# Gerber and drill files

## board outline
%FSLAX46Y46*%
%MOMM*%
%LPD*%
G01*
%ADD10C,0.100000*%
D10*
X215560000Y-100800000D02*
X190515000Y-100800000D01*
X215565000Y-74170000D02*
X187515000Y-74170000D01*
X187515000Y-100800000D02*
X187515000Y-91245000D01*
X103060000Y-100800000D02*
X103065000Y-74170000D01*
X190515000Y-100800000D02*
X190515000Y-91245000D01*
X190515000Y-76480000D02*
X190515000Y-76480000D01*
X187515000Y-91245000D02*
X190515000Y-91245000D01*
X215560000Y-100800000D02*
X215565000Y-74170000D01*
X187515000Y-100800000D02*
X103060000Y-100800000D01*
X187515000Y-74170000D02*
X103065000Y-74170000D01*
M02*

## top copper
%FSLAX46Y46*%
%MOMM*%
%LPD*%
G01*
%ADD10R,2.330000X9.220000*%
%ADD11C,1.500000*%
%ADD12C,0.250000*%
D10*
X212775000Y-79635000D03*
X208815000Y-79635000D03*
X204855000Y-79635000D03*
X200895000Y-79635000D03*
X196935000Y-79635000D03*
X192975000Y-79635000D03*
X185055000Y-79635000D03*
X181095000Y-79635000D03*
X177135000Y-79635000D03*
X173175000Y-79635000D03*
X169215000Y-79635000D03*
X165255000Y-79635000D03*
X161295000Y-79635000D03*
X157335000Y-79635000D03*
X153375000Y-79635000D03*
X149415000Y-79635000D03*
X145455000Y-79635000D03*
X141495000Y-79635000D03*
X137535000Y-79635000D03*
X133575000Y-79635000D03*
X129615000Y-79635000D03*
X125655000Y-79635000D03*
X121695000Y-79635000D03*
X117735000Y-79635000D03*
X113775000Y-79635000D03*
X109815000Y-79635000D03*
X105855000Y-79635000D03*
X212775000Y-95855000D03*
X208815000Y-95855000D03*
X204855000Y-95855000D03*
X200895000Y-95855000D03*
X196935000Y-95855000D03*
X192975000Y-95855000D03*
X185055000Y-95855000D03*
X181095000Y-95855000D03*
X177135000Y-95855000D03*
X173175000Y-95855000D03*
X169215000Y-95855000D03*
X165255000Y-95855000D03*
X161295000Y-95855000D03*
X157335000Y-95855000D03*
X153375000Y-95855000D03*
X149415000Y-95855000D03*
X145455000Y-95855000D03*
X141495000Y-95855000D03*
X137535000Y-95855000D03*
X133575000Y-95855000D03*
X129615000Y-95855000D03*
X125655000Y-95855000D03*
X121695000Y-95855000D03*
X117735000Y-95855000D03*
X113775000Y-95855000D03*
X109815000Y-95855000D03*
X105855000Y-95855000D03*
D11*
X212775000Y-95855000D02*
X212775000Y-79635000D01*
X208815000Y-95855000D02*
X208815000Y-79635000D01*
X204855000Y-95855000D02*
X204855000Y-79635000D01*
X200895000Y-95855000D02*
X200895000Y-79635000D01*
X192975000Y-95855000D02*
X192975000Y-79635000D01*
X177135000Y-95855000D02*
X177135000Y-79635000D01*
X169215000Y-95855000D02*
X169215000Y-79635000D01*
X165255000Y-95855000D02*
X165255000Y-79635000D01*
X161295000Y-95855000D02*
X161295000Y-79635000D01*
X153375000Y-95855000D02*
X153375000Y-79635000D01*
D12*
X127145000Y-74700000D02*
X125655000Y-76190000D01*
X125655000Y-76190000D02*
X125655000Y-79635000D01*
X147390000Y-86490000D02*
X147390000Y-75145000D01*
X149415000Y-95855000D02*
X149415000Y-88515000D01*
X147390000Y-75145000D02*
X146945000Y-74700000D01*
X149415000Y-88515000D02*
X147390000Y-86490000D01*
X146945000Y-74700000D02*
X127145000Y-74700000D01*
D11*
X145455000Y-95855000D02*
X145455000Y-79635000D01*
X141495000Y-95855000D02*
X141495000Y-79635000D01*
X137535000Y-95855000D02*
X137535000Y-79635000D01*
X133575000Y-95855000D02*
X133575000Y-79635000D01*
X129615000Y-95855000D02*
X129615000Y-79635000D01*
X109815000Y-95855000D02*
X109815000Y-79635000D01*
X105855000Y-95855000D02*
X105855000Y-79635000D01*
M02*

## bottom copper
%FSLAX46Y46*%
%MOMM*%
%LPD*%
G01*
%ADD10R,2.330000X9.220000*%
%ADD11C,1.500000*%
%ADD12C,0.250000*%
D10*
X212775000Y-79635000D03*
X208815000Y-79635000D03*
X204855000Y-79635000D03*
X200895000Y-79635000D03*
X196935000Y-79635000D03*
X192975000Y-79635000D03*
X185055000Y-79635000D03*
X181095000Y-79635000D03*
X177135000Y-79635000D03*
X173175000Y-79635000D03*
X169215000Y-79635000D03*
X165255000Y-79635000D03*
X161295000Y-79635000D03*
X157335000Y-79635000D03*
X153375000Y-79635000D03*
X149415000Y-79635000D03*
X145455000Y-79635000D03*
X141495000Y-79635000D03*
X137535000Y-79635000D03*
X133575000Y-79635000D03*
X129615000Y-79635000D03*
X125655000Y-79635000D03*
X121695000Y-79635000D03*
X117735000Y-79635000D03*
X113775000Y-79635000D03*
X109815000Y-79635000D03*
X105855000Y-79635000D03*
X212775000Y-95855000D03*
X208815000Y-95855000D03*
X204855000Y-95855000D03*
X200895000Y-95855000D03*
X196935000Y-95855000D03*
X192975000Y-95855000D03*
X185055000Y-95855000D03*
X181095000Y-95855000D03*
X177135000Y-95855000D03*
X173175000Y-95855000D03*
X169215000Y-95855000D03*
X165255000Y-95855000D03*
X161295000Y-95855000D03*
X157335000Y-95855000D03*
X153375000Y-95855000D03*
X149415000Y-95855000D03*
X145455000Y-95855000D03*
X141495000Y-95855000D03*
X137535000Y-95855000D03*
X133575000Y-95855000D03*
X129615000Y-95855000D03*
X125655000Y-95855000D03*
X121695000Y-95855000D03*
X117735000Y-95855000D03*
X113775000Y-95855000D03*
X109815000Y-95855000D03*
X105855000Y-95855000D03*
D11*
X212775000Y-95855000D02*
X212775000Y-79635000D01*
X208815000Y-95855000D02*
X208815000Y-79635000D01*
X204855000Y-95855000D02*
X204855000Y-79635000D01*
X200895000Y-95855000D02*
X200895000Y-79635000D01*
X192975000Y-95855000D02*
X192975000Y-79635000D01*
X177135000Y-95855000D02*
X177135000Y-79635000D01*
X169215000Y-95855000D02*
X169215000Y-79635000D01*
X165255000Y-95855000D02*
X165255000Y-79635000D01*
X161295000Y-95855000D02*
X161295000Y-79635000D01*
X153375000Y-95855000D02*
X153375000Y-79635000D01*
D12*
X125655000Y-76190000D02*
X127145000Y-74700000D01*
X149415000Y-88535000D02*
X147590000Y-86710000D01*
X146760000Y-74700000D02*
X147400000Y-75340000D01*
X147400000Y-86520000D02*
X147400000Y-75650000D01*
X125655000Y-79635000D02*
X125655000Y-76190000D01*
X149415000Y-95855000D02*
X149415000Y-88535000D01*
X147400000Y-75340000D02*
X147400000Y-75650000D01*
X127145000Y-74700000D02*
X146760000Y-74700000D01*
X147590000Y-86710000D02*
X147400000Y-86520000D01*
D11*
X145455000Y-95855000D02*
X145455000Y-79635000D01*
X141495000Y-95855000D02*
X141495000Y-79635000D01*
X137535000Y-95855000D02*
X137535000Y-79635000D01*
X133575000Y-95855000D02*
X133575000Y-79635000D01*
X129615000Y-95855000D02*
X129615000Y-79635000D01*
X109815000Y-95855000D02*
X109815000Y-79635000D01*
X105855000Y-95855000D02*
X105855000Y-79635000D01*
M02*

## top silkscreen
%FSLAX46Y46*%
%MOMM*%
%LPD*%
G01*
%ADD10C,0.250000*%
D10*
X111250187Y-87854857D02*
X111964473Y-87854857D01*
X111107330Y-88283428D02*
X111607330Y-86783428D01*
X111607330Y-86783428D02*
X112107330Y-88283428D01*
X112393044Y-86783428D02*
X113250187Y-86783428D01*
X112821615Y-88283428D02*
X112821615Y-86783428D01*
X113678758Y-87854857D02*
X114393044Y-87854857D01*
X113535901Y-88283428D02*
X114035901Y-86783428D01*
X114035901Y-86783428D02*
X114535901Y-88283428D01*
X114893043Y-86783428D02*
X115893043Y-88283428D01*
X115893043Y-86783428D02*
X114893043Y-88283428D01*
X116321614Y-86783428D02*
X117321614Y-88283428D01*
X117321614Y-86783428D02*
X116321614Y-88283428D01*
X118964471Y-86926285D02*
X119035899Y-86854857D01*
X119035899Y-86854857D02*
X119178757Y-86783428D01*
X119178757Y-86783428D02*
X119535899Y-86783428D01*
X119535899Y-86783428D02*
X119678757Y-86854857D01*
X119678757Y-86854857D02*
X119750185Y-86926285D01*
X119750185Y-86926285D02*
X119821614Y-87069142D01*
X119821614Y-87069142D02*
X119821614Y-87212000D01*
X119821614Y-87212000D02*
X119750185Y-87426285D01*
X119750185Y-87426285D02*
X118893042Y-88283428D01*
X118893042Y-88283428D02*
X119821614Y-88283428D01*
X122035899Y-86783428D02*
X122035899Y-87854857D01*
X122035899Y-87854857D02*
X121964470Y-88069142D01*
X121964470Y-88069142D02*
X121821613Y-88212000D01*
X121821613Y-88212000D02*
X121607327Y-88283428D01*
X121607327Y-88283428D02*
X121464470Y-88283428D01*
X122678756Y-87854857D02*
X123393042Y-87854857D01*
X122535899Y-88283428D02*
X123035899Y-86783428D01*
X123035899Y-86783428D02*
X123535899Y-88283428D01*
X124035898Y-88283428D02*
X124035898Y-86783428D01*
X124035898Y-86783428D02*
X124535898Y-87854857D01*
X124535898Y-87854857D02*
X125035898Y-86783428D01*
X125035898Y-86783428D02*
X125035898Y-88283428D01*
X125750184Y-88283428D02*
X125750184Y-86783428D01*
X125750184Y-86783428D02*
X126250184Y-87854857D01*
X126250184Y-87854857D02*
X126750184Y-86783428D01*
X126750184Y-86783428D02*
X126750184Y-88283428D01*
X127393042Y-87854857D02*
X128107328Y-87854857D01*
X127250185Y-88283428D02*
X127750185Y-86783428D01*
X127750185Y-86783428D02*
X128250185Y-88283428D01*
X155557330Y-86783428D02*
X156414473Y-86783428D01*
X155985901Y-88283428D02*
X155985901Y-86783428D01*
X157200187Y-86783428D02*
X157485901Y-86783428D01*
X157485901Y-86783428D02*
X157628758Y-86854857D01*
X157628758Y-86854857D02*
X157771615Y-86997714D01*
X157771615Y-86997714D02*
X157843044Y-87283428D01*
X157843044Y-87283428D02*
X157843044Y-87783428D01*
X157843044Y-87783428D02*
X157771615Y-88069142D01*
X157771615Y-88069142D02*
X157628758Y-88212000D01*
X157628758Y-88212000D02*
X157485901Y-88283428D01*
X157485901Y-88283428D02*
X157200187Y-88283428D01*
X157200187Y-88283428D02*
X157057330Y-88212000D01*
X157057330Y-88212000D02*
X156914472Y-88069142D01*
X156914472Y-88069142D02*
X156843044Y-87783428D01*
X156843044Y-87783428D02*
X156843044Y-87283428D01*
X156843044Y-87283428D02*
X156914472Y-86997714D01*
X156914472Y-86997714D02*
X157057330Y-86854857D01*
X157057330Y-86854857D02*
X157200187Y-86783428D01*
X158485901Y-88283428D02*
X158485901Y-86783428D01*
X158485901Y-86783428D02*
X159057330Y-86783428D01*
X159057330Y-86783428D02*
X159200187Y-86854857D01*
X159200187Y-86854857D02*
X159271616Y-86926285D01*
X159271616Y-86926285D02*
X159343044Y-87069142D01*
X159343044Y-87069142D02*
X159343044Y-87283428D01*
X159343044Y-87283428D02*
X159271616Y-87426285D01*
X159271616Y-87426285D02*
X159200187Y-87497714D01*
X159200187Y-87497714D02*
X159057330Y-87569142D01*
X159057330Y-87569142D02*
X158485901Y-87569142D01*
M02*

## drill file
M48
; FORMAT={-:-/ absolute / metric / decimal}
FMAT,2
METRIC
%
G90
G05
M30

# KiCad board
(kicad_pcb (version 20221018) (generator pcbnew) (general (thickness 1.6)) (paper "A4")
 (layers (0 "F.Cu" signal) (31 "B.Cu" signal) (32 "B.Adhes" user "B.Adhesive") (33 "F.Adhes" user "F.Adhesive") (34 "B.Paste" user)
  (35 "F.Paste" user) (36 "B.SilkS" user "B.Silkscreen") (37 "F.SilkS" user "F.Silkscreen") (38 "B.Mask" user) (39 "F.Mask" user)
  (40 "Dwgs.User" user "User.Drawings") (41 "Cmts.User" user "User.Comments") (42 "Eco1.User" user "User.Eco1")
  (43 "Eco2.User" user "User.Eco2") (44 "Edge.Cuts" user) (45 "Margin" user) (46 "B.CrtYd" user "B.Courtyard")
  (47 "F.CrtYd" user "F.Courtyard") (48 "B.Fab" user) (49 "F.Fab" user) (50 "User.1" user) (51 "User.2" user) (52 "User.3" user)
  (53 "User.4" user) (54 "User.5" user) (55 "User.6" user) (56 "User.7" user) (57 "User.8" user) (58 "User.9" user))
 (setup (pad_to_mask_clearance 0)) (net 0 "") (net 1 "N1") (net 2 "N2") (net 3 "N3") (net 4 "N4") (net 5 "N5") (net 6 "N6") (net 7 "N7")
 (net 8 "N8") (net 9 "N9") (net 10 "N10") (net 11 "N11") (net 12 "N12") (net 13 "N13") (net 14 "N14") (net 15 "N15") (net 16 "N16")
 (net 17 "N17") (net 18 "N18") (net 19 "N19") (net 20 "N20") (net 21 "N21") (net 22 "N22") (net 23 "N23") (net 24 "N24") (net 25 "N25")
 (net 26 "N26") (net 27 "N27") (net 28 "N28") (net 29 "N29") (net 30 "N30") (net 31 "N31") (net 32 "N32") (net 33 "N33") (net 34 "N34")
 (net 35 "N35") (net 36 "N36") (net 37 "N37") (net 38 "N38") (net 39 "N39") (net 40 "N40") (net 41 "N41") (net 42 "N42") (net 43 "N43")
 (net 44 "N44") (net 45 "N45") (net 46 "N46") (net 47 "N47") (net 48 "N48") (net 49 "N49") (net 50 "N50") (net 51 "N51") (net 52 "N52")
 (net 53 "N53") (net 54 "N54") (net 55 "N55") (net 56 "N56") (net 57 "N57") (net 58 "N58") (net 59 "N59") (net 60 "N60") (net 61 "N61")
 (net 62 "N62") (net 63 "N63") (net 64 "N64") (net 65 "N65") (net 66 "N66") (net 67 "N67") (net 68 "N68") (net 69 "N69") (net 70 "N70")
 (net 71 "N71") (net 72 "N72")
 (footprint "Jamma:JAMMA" (layer "F.Cu") (at 159.435 79.635 180)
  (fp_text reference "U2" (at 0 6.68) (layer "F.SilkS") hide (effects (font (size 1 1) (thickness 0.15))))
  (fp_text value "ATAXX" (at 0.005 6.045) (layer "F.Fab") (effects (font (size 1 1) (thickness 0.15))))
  (pad "1" smd rect (at -53.34 0 180) (size 2.33 9.22) (layers "F.Cu" "F.Paste" "F.Mask") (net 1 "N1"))
  (pad "2" smd rect (at -49.38 0 180) (size 2.33 9.22) (layers "F.Cu" "F.Paste" "F.Mask") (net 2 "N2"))
  (pad "3" smd rect (at -45.42 0 180) (size 2.33 9.22) (layers "F.Cu" "F.Paste" "F.Mask") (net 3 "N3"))
  (pad "4" smd rect (at -41.46 0 180) (size 2.33 9.22) (layers "F.Cu" "F.Paste" "F.Mask") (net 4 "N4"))
  (pad "5" smd rect (at -37.5 0 180) (size 2.33 9.22) (layers "F.Cu" "F.Paste" "F.Mask") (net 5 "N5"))
  (pad "6" smd rect (at -33.54 0 180) (size 2.33 9.22) (layers "F.Cu" "F.Paste" "F.Mask") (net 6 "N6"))
  (pad "8" smd rect (at -25.62 0 180) (size 2.33 9.22) (layers "F.Cu" "F.Paste" "F.Mask") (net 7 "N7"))
  (pad "9" smd rect (at -21.66 0 180) (size 2.33 9.22) (layers "F.Cu" "F.Paste" "F.Mask") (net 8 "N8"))
  (pad "10" smd rect (at -17.7 0 180) (size 2.33 9.22) (layers "F.Cu" "F.Paste" "F.Mask") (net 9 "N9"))
  (pad "11" smd rect (at -13.74 0 180) (size 2.33 9.22) (layers "F.Cu" "F.Paste" "F.Mask") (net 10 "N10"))
  (pad "12" smd rect (at -9.78 0 180) (size 2.33 9.22) (layers "F.Cu" "F.Paste" "F.Mask") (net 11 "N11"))
  (pad "13" smd rect (at -5.82 0 180) (size 2.33 9.22) (layers "F.Cu" "F.Paste" "F.Mask") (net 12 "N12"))
  (pad "14" smd rect (at -1.86 0 180) (size 2.33 9.22) (layers "F.Cu" "F.Paste" "F.Mask") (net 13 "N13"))
  (pad "15" smd rect (at 2.1 0 180) (size 2.33 9.22) (layers "F.Cu" "F.Paste" "F.Mask") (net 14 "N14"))
  (pad "16" smd rect (at 6.06 0 180) (size 2.33 9.22) (layers "F.Cu" "F.Paste" "F.Mask") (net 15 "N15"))
  (pad "17" smd rect (at 10.02 0 180) (size 2.33 9.22) (layers "F.Cu" "F.Paste" "F.Mask") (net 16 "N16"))
  (pad "18" smd rect (at 13.98 0 180) (size 2.33 9.22) (layers "F.Cu" "F.Paste" "F.Mask") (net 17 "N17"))
  (pad "19" smd rect (at 17.94 0 180) (size 2.33 9.22) (layers "F.Cu" "F.Paste" "F.Mask") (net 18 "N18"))
  (pad "20" smd rect (at 21.9 0 180) (size 2.33 9.22) (layers "F.Cu" "F.Paste" "F.Mask") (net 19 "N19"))
  (pad "21" smd rect (at 25.86 0 180) (size 2.33 9.22) (layers "F.Cu" "F.Paste" "F.Mask") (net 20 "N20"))
  (pad "22" smd rect (at 29.82 0 180) (size 2.33 9.22) (layers "F.Cu" "F.Paste" "F.Mask") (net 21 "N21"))
  (pad "23" smd rect (at 33.78 0 180) (size 2.33 9.22) (layers "F.Cu" "F.Paste" "F.Mask") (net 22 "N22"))
  (pad "24" smd rect (at 37.74 0 180) (size 2.33 9.22) (layers "F.Cu" "F.Paste" "F.Mask") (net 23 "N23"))
  (pad "25" smd rect (at 41.7 0 180) (size 2.33 9.22) (layers "F.Cu" "F.Paste" "F.Mask") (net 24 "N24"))
  (pad "26" smd rect (at 45.66 0 180) (size 2.33 9.22) (layers "F.Cu" "F.Paste" "F.Mask") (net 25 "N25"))
  (pad "27" smd rect (at 49.62 0 180) (size 2.33 9.22) (layers "F.Cu" "F.Paste" "F.Mask") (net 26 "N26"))
  (pad "28" smd rect (at 53.58 0 180) (size 2.33 9.22) (layers "F.Cu" "F.Paste" "F.Mask") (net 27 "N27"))
  (pad "A" smd rect (at -53.34 0 180) (size 2.33 9.22) (layers "B.Cu" "B.Paste" "B.Mask") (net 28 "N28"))
  (pad "B" smd rect (at -49.38 0 180) (size 2.33 9.22) (layers "B.Cu" "B.Paste" "B.Mask") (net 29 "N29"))
  (pad "C" smd rect (at -45.42 0 180) (size 2.33 9.22) (layers "B.Cu" "B.Paste" "B.Mask") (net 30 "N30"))
  (pad "D" smd rect (at -41.46 0 180) (size 2.33 9.22) (layers "B.Cu" "B.Paste" "B.Mask") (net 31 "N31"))
  (pad "E" smd rect (at -37.5 0 180) (size 2.33 9.22) (layers "B.Cu" "B.Paste" "B.Mask") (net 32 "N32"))
  (pad "F" smd rect (at -33.54 0 180) (size 2.33 9.22) (layers "B.Cu" "B.Paste" "B.Mask") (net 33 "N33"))
  (pad "J" smd rect (at -25.62 0 180) (size 2.33 9.22) (layers "B.Cu" "B.Paste" "B.Mask") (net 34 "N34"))
  (pad "K" smd rect (at -21.66 0 180) (size 2.33 9.22) (layers "B.Cu" "B.Paste" "B.Mask") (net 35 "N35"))
  (pad "L" smd rect (at -17.7 0 180) (size 2.33 9.22) (layers "B.Cu" "B.Paste" "B.Mask") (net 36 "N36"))
  (pad "M" smd rect (at -13.74 0 180) (size 2.33 9.22) (layers "B.Cu" "B.Paste" "B.Mask") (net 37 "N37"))
  (pad "N" smd rect (at -9.78 0 180) (size 2.33 9.22) (layers "B.Cu" "B.Paste" "B.Mask") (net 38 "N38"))
  (pad "P" smd rect (at -5.82 0 180) (size 2.33 9.22) (layers "B.Cu" "B.Paste" "B.Mask") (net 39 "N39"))
  (pad "R" smd rect (at -1.86 0 180) (size 2.33 9.22) (layers "B.Cu" "B.Paste" "B.Mask") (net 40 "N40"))
  (pad "S" smd rect (at 2.1 0 180) (size 2.33 9.22) (layers "B.Cu" "B.Paste" "B.Mask") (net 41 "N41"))
  (pad "T" smd rect (at 6.06 0 180) (size 2.33 9.22) (layers "B.Cu" "B.Paste" "B.Mask") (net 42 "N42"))
  (pad "U" smd rect (at 10.02 0 180) (size 2.33 9.22) (layers "B.Cu" "B.Paste" "B.Mask") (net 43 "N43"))
  (pad "V" smd rect (at 13.98 0 180) (size 2.33 9.22) (layers "B.Cu" "B.Paste" "B.Mask") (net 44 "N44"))
  (pad "W" smd rect (at 17.94 0 180) (size 2.33 9.22) (layers "B.Cu" "B.Paste" "B.Mask") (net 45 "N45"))
  (pad "X" smd rect (at 21.9 0 180) (size 2.33 9.22) (layers "B.Cu" "B.Paste" "B.Mask") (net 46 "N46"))
  (pad "Y" smd rect (at 25.86 0 180) (size 2.33 9.22) (layers "B.Cu" "B.Paste" "B.Mask") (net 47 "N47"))
  (pad "Z" smd rect (at 29.82 0 180) (size 2.33 9.22) (layers "B.Cu" "B.Paste" "B.Mask") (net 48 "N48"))
  (pad "a" smd rect (at 33.78 0 180) (size 2.33 9.22) (layers "B.Cu" "B.Paste" "B.Mask") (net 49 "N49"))
  (pad "b" smd rect (at 37.74 0 180) (size 2.33 9.22) (layers "B.Cu" "B.Paste" "B.Mask") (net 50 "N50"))
  (pad "c" smd rect (at 41.7 0 180) (size 2.33 9.22) (layers "B.Cu" "B.Paste" "B.Mask") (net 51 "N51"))
  (pad "d" smd rect (at 45.66 0 180) (size 2.33 9.22) (layers "B.Cu" "B.Paste" "B.Mask") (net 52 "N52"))
  (pad "e" smd rect (at 49.62 0 180) (size 2.33 9.22) (layers "B.Cu" "B.Paste" "B.Mask") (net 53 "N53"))
  (pad "f" smd rect (at 53.58 0 180) (size 2.33 9.22) (layers "B.Cu" "B.Paste" "B.Mask") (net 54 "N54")))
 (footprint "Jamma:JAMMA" (layer "F.Cu") (at 159.435 95.855 180)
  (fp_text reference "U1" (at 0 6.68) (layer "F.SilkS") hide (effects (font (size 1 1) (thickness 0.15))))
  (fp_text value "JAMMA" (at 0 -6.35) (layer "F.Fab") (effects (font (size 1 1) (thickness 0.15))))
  (pad "1" smd rect (at -53.34 0 180) (size 2.33 9.22) (layers "F.Cu" "F.Paste" "F.Mask") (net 1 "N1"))
  (pad "2" smd rect (at -49.38 0 180) (size 2.33 9.22) (layers "F.Cu" "F.Paste" "F.Mask") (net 2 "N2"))
  (pad "3" smd rect (at -45.42 0 180) (size 2.33 9.22) (layers "F.Cu" "F.Paste" "F.Mask") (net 3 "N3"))
  (pad "4" smd rect (at -41.46 0 180) (size 2.33 9.22) (layers "F.Cu" "F.Paste" "F.Mask") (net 4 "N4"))
  (pad "5" smd rect (at -37.5 0 180) (size 2.33 9.22) (layers "F.Cu" "F.Paste" "F.Mask") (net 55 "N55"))
  (pad "6" smd rect (at -33.54 0 180) (size 2.33 9.22) (layers "F.Cu" "F.Paste" "F.Mask") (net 6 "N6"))
  (pad "8" smd rect (at -25.62 0 180) (size 2.33 9.22) (layers "F.Cu" "F.Paste" "F.Mask") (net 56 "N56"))
  (pad "9" smd rect (at -21.66 0 180) (size 2.33 9.22) (layers "F.Cu" "F.Paste" "F.Mask") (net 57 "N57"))
  (pad "10" smd rect (at -17.7 0 180) (size 2.33 9.22) (layers "F.Cu" "F.Paste" "F.Mask") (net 9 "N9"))
  (pad "11" smd rect (at -13.74 0 180) (size 2.33 9.22) (layers "F.Cu" "F.Paste" "F.Mask") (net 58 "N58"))
  (pad "12" smd rect (at -9.78 0 180) (size 2.33 9.22) (layers "F.Cu" "F.Paste" "F.Mask") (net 11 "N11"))
  (pad "13" smd rect (at -5.82 0 180) (size 2.33 9.22) (layers "F.Cu" "F.Paste" "F.Mask") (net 12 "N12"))
  (pad "14" smd rect (at -1.86 0 180) (size 2.33 9.22) (layers "F.Cu" "F.Paste" "F.Mask") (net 13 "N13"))
  (pad "15" smd rect (at 2.1 0 180) (size 2.33 9.22) (layers "F.Cu" "F.Paste" "F.Mask") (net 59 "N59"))
  (pad "16" smd rect (at 6.06 0 180) (size 2.33 9.22) (layers "F.Cu" "F.Paste" "F.Mask") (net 15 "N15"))
  (pad "17" smd rect (at 10.02 0 180) (size 2.33 9.22) (layers "F.Cu" "F.Paste" "F.Mask") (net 22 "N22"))
  (pad "18" smd rect (at 13.98 0 180) (size 2.33 9.22) (layers "F.Cu" "F.Paste" "F.Mask") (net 17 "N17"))
  (pad "19" smd rect (at 17.94 0 180) (size 2.33 9.22) (layers "F.Cu" "F.Paste" "F.Mask") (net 18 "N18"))
  (pad "20" smd rect (at 21.9 0 180) (size 2.33 9.22) (layers "F.Cu" "F.Paste" "F.Mask") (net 19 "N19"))
  (pad "21" smd rect (at 25.86 0 180) (size 2.33 9.22) (layers "F.Cu" "F.Paste" "F.Mask") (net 20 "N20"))
  (pad "22" smd rect (at 29.82 0 180) (size 2.33 9.22) (layers "F.Cu" "F.Paste" "F.Mask") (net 21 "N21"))
  (pad "23" smd rect (at 33.78 0 180) (size 2.33 9.22) (layers "F.Cu" "F.Paste" "F.Mask") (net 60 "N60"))
  (pad "24" smd rect (at 37.74 0 180) (size 2.33 9.22) (layers "F.Cu" "F.Paste" "F.Mask") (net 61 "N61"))
  (pad "25" smd rect (at 41.7 0 180) (size 2.33 9.22) (layers "F.Cu" "F.Paste" "F.Mask") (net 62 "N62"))
  (pad "26" smd rect (at 45.66 0 180) (size 2.33 9.22) (layers "F.Cu" "F.Paste" "F.Mask") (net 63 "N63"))
  (pad "27" smd rect (at 49.62 0 180) (size 2.33 9.22) (layers "F.Cu" "F.Paste" "F.Mask") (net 26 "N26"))
  (pad "28" smd rect (at 53.58 0 180) (size 2.33 9.22) (layers "F.Cu" "F.Paste" "F.Mask") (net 27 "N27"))
  (pad "A" smd rect (at -53.34 0 180) (size 2.33 9.22) (layers "B.Cu" "B.Paste" "B.Mask") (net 28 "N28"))
  (pad "B" smd rect (at -49.38 0 180) (size 2.33 9.22) (layers "B.Cu" "B.Paste" "B.Mask") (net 29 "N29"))
  (pad "C" smd rect (at -45.42 0 180) (size 2.33 9.22) (layers "B.Cu" "B.Paste" "B.Mask") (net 30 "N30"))
  (pad "D" smd rect (at -41.46 0 180) (size 2.33 9.22) (layers "B.Cu" "B.Paste" "B.Mask") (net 31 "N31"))
  (pad "E" smd rect (at -37.5 0 180) (size 2.33 9.22) (layers "B.Cu" "B.Paste" "B.Mask") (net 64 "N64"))
  (pad "F" smd rect (at -33.54 0 180) (size 2.33 9.22) (layers "B.Cu" "B.Paste" "B.Mask") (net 33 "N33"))
  (pad "J" smd rect (at -25.62 0 180) (size 2.33 9.22) (layers "B.Cu" "B.Paste" "B.Mask") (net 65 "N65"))
  (pad "K" smd rect (at -21.66 0 180) (size 2.33 9.22) (layers "B.Cu" "B.Paste" "B.Mask") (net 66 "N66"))
  (pad "L" smd rect (at -17.7 0 180) (size 2.33 9.22) (layers "B.Cu" "B.Paste" "B.Mask") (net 36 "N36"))
  (pad "M" smd rect (at -13.74 0 180) (size 2.33 9.22) (layers "B.Cu" "B.Paste" "B.Mask") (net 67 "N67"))
  (pad "N" smd rect (at -9.78 0 180) (size 2.33 9.22) (layers "B.Cu" "B.Paste" "B.Mask") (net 38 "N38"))
  (pad "P" smd rect (at -5.82 0 180) (size 2.33 9.22) (layers "B.Cu" "B.Paste" "B.Mask") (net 39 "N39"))
  (pad "R" smd rect (at -1.86 0 180) (size 2.33 9.22) (layers "B.Cu" "B.Paste" "B.Mask") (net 40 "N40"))
  (pad "S" smd rect (at 2.1 0 180) (size 2.33 9.22) (layers "B.Cu" "B.Paste" "B.Mask") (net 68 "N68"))
  (pad "T" smd rect (at 6.06 0 180) (size 2.33 9.22) (layers "B.Cu" "B.Paste" "B.Mask") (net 42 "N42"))
  (pad "U" smd rect (at 10.02 0 180) (size 2.33 9.22) (layers "B.Cu" "B.Paste" "B.Mask") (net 49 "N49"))
  (pad "V" smd rect (at 13.98 0 180) (size 2.33 9.22) (layers "B.Cu" "B.Paste" "B.Mask") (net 44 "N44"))
  (pad "W" smd rect (at 17.94 0 180) (size 2.33 9.22) (layers "B.Cu" "B.Paste" "B.Mask") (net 45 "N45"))
  (pad "X" smd rect (at 21.9 0 180) (size 2.33 9.22) (layers "B.Cu" "B.Paste" "B.Mask") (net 46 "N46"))
  (pad "Y" smd rect (at 25.86 0 180) (size 2.33 9.22) (layers "B.Cu" "B.Paste" "B.Mask") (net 47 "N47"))
  (pad "Z" smd rect (at 29.82 0 180) (size 2.33 9.22) (layers "B.Cu" "B.Paste" "B.Mask") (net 48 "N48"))
  (pad "a" smd rect (at 33.78 0 180) (size 2.33 9.22) (layers "B.Cu" "B.Paste" "B.Mask") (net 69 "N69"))
  (pad "b" smd rect (at 37.74 0 180) (size 2.33 9.22) (layers "B.Cu" "B.Paste" "B.Mask") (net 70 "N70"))
  (pad "c" smd rect (at 41.7 0 180) (size 2.33 9.22) (layers "B.Cu" "B.Paste" "B.Mask") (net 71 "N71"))
  (pad "d" smd rect (at 45.66 0 180) (size 2.33 9.22) (layers "B.Cu" "B.Paste" "B.Mask") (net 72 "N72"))
  (pad "e" smd rect (at 49.62 0 180) (size 2.33 9.22) (layers "B.Cu" "B.Paste" "B.Mask") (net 53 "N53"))
  (pad "f" smd rect (at 53.58 0 180) (size 2.33 9.22) (layers "B.Cu" "B.Paste" "B.Mask") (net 54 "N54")))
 (gr_line (start 215.56 100.8) (end 190.515 100.8) (stroke (width 0.1) (type default)) (layer "Edge.Cuts"))
 (gr_line (start 215.565 74.17) (end 187.515 74.17) (stroke (width 0.1) (type default)) (layer "Edge.Cuts"))
 (gr_line (start 187.515 100.8) (end 187.515 91.245) (stroke (width 0.1) (type default)) (layer "Edge.Cuts"))
 (gr_line (start 103.06 100.8) (end 103.065 74.17) (stroke (width 0.1) (type default)) (layer "Edge.Cuts"))
 (gr_line (start 190.515 100.8) (end 190.515 91.245) (stroke (width 0.1) (type default)) (layer "Edge.Cuts"))
 (gr_line (start 190.515 76.48) (end 190.515 76.48) (stroke (width 0.1) (type default)) (layer "Edge.Cuts"))
 (gr_line (start 187.515 91.245) (end 190.515 91.245) (stroke (width 0.1) (type default)) (layer "Edge.Cuts"))
 (gr_line (start 215.56 100.8) (end 215.565 74.17) (stroke (width 0.1) (type default)) (layer "Edge.Cuts"))
 (gr_line (start 187.515 100.8) (end 103.06 100.8) (stroke (width 0.1) (type default)) (layer "Edge.Cuts"))
 (gr_line (start 187.515 74.17) (end 103.065 74.17) (stroke (width 0.1) (type default)) (layer "Edge.Cuts"))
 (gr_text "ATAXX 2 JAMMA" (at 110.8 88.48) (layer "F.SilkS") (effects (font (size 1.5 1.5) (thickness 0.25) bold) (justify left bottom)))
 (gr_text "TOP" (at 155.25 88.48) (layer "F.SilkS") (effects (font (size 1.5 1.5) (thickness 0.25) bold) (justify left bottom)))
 (segment (start 212.775 95.855) (end 212.775 79.635) (width 1.5) (layer "F.Cu") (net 1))
 (segment (start 208.815 95.855) (end 208.815 79.635) (width 1.5) (layer "F.Cu") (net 2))
 (segment (start 204.855 95.855) (end 204.855 79.635) (width 1.5) (layer "F.Cu") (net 3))
 (segment (start 200.895 95.855) (end 200.895 79.635) (width 1.5) (layer "F.Cu") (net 4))
 (segment (start 192.975 95.855) (end 192.975 79.635) (width 1.5) (layer "F.Cu") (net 6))
 (segment (start 177.135 95.855) (end 177.135 79.635) (width 1.5) (layer "F.Cu") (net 9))
 (segment (start 169.215 95.855) (end 169.215 79.635) (width 1.5) (layer "F.Cu") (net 11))
 (segment (start 165.255 95.855) (end 165.255 79.635) (width 1.5) (layer "F.Cu") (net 12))
 (segment (start 161.295 95.855) (end 161.295 79.635) (width 1.5) (layer "F.Cu") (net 13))
 (segment (start 153.375 95.855) (end 153.375 79.635) (width 1.5) (layer "F.Cu") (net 15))
 (segment (start 127.145 74.7) (end 125.655 76.19) (width 0.25) (layer "F.Cu") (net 22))
 (segment (start 125.655 76.19) (end 125.655 79.635) (width 0.25) (layer "F.Cu") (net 22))
 (segment (start 147.39 86.49) (end 147.39 75.145) (width 0.25) (layer "F.Cu") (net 22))
 (segment (start 149.415 95.855) (end 149.415 88.515) (width 0.25) (layer "F.Cu") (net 22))
 (segment (start 147.39 75.145) (end 146.945 74.7) (width 0.25) (layer "F.Cu") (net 22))
 (segment (start 149.415 88.515) (end 147.39 86.49) (width 0.25) (layer "F.Cu") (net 22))
 (segment (start 146.945 74.7) (end 127.145 74.7) (width 0.25) (layer "F.Cu") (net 22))
 (segment (start 145.455 95.855) (end 145.455 79.635) (width 1.5) (layer "F.Cu") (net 17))
 (segment (start 141.495 95.855) (end 141.495 79.635) (width 1.5) (layer "F.Cu") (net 18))
 (segment (start 137.535 95.855) (end 137.535 79.635) (width 1.5) (layer "F.Cu") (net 19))
 (segment (start 133.575 95.855) (end 133.575 79.635) (width 1.5) (layer "F.Cu") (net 20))
 (segment (start 129.615 95.855) (end 129.615 79.635) (width 1.5) (layer "F.Cu") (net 21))
 (segment (start 109.815 95.855) (end 109.815 79.635) (width 1.5) (layer "F.Cu") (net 26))
 (segment (start 105.855 95.855) (end 105.855 79.635) (width 1.5) (layer "F.Cu") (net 27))
 (segment (start 212.775 95.855) (end 212.775 79.635) (width 1.5) (layer "B.Cu") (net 28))
 (segment (start 208.815 95.855) (end 208.815 79.635) (width 1.5) (layer "B.Cu") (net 29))
 (segment (start 204.855 95.855) (end 204.855 79.635) (width 1.5) (layer "B.Cu") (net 30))
 (segment (start 200.895 95.855) (end 200.895 79.635) (width 1.5) (layer "B.Cu") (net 31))
 (segment (start 192.975 95.855) (end 192.975 79.635) (width 1.5) (layer "B.Cu") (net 33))
 (segment (start 177.135 95.855) (end 177.135 79.635) (width 1.5) (layer "B.Cu") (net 36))
 (segment (start 169.215 95.855) (end 169.215 79.635) (width 1.5) (layer "B.Cu") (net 38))
 (segment (start 165.255 95.855) (end 165.255 79.635) (width 1.5) (layer "B.Cu") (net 39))
 (segment (start 161.295 95.855) (end 161.295 79.635) (width 1.5) (layer "B.Cu") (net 40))
 (segment (start 153.375 95.855) (end 153.375 79.635) (width 1.5) (layer "B.Cu") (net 42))
 (segment (start 125.655 76.19) (end 127.145 74.7) (width 0.25) (layer "B.Cu") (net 49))
 (segment (start 149.415 88.535) (end 147.59 86.71) (width 0.25) (layer "B.Cu") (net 49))
 (segment (start 146.76 74.7) (end 147.4 75.34) (width 0.25) (layer "B.Cu") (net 49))
 (segment (start 147.4 86.52) (end 147.4 75.65) (width 0.25) (layer "B.Cu") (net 49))
 (segment (start 125.655 79.635) (end 125.655 76.19) (width 0.25) (layer "B.Cu") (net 49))
 (segment (start 149.415 95.855) (end 149.415 88.535) (width 0.25) (layer "B.Cu") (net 49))
 (segment (start 147.4 75.34) (end 147.4 75.65) (width 0.25) (layer "B.Cu") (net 49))
 (segment (start 127.145 74.7) (end 146.76 74.7) (width 0.25) (layer "B.Cu") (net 49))
 (segment (start 147.59 86.71) (end 147.4 86.52) (width 0.25) (layer "B.Cu") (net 49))
 (segment (start 145.455 95.855) (end 145.455 79.635) (width 1.5) (layer "B.Cu") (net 44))
 (segment (start 141.495 95.855) (end 141.495 79.635) (width 1.5) (layer "B.Cu") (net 45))
 (segment (start 137.535 95.855) (end 137.535 79.635) (width 1.5) (layer "B.Cu") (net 46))
 (segment (start 133.575 95.855) (end 133.575 79.635) (width 1.5) (layer "B.Cu") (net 47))
 (segment (start 129.615 95.855) (end 129.615 79.635) (width 1.5) (layer "B.Cu") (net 48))
 (segment (start 109.815 95.855) (end 109.815 79.635) (width 1.5) (layer "B.Cu") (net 53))
 (segment (start 105.855 95.855) (end 105.855 79.635) (width 1.5) (layer "B.Cu") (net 54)))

